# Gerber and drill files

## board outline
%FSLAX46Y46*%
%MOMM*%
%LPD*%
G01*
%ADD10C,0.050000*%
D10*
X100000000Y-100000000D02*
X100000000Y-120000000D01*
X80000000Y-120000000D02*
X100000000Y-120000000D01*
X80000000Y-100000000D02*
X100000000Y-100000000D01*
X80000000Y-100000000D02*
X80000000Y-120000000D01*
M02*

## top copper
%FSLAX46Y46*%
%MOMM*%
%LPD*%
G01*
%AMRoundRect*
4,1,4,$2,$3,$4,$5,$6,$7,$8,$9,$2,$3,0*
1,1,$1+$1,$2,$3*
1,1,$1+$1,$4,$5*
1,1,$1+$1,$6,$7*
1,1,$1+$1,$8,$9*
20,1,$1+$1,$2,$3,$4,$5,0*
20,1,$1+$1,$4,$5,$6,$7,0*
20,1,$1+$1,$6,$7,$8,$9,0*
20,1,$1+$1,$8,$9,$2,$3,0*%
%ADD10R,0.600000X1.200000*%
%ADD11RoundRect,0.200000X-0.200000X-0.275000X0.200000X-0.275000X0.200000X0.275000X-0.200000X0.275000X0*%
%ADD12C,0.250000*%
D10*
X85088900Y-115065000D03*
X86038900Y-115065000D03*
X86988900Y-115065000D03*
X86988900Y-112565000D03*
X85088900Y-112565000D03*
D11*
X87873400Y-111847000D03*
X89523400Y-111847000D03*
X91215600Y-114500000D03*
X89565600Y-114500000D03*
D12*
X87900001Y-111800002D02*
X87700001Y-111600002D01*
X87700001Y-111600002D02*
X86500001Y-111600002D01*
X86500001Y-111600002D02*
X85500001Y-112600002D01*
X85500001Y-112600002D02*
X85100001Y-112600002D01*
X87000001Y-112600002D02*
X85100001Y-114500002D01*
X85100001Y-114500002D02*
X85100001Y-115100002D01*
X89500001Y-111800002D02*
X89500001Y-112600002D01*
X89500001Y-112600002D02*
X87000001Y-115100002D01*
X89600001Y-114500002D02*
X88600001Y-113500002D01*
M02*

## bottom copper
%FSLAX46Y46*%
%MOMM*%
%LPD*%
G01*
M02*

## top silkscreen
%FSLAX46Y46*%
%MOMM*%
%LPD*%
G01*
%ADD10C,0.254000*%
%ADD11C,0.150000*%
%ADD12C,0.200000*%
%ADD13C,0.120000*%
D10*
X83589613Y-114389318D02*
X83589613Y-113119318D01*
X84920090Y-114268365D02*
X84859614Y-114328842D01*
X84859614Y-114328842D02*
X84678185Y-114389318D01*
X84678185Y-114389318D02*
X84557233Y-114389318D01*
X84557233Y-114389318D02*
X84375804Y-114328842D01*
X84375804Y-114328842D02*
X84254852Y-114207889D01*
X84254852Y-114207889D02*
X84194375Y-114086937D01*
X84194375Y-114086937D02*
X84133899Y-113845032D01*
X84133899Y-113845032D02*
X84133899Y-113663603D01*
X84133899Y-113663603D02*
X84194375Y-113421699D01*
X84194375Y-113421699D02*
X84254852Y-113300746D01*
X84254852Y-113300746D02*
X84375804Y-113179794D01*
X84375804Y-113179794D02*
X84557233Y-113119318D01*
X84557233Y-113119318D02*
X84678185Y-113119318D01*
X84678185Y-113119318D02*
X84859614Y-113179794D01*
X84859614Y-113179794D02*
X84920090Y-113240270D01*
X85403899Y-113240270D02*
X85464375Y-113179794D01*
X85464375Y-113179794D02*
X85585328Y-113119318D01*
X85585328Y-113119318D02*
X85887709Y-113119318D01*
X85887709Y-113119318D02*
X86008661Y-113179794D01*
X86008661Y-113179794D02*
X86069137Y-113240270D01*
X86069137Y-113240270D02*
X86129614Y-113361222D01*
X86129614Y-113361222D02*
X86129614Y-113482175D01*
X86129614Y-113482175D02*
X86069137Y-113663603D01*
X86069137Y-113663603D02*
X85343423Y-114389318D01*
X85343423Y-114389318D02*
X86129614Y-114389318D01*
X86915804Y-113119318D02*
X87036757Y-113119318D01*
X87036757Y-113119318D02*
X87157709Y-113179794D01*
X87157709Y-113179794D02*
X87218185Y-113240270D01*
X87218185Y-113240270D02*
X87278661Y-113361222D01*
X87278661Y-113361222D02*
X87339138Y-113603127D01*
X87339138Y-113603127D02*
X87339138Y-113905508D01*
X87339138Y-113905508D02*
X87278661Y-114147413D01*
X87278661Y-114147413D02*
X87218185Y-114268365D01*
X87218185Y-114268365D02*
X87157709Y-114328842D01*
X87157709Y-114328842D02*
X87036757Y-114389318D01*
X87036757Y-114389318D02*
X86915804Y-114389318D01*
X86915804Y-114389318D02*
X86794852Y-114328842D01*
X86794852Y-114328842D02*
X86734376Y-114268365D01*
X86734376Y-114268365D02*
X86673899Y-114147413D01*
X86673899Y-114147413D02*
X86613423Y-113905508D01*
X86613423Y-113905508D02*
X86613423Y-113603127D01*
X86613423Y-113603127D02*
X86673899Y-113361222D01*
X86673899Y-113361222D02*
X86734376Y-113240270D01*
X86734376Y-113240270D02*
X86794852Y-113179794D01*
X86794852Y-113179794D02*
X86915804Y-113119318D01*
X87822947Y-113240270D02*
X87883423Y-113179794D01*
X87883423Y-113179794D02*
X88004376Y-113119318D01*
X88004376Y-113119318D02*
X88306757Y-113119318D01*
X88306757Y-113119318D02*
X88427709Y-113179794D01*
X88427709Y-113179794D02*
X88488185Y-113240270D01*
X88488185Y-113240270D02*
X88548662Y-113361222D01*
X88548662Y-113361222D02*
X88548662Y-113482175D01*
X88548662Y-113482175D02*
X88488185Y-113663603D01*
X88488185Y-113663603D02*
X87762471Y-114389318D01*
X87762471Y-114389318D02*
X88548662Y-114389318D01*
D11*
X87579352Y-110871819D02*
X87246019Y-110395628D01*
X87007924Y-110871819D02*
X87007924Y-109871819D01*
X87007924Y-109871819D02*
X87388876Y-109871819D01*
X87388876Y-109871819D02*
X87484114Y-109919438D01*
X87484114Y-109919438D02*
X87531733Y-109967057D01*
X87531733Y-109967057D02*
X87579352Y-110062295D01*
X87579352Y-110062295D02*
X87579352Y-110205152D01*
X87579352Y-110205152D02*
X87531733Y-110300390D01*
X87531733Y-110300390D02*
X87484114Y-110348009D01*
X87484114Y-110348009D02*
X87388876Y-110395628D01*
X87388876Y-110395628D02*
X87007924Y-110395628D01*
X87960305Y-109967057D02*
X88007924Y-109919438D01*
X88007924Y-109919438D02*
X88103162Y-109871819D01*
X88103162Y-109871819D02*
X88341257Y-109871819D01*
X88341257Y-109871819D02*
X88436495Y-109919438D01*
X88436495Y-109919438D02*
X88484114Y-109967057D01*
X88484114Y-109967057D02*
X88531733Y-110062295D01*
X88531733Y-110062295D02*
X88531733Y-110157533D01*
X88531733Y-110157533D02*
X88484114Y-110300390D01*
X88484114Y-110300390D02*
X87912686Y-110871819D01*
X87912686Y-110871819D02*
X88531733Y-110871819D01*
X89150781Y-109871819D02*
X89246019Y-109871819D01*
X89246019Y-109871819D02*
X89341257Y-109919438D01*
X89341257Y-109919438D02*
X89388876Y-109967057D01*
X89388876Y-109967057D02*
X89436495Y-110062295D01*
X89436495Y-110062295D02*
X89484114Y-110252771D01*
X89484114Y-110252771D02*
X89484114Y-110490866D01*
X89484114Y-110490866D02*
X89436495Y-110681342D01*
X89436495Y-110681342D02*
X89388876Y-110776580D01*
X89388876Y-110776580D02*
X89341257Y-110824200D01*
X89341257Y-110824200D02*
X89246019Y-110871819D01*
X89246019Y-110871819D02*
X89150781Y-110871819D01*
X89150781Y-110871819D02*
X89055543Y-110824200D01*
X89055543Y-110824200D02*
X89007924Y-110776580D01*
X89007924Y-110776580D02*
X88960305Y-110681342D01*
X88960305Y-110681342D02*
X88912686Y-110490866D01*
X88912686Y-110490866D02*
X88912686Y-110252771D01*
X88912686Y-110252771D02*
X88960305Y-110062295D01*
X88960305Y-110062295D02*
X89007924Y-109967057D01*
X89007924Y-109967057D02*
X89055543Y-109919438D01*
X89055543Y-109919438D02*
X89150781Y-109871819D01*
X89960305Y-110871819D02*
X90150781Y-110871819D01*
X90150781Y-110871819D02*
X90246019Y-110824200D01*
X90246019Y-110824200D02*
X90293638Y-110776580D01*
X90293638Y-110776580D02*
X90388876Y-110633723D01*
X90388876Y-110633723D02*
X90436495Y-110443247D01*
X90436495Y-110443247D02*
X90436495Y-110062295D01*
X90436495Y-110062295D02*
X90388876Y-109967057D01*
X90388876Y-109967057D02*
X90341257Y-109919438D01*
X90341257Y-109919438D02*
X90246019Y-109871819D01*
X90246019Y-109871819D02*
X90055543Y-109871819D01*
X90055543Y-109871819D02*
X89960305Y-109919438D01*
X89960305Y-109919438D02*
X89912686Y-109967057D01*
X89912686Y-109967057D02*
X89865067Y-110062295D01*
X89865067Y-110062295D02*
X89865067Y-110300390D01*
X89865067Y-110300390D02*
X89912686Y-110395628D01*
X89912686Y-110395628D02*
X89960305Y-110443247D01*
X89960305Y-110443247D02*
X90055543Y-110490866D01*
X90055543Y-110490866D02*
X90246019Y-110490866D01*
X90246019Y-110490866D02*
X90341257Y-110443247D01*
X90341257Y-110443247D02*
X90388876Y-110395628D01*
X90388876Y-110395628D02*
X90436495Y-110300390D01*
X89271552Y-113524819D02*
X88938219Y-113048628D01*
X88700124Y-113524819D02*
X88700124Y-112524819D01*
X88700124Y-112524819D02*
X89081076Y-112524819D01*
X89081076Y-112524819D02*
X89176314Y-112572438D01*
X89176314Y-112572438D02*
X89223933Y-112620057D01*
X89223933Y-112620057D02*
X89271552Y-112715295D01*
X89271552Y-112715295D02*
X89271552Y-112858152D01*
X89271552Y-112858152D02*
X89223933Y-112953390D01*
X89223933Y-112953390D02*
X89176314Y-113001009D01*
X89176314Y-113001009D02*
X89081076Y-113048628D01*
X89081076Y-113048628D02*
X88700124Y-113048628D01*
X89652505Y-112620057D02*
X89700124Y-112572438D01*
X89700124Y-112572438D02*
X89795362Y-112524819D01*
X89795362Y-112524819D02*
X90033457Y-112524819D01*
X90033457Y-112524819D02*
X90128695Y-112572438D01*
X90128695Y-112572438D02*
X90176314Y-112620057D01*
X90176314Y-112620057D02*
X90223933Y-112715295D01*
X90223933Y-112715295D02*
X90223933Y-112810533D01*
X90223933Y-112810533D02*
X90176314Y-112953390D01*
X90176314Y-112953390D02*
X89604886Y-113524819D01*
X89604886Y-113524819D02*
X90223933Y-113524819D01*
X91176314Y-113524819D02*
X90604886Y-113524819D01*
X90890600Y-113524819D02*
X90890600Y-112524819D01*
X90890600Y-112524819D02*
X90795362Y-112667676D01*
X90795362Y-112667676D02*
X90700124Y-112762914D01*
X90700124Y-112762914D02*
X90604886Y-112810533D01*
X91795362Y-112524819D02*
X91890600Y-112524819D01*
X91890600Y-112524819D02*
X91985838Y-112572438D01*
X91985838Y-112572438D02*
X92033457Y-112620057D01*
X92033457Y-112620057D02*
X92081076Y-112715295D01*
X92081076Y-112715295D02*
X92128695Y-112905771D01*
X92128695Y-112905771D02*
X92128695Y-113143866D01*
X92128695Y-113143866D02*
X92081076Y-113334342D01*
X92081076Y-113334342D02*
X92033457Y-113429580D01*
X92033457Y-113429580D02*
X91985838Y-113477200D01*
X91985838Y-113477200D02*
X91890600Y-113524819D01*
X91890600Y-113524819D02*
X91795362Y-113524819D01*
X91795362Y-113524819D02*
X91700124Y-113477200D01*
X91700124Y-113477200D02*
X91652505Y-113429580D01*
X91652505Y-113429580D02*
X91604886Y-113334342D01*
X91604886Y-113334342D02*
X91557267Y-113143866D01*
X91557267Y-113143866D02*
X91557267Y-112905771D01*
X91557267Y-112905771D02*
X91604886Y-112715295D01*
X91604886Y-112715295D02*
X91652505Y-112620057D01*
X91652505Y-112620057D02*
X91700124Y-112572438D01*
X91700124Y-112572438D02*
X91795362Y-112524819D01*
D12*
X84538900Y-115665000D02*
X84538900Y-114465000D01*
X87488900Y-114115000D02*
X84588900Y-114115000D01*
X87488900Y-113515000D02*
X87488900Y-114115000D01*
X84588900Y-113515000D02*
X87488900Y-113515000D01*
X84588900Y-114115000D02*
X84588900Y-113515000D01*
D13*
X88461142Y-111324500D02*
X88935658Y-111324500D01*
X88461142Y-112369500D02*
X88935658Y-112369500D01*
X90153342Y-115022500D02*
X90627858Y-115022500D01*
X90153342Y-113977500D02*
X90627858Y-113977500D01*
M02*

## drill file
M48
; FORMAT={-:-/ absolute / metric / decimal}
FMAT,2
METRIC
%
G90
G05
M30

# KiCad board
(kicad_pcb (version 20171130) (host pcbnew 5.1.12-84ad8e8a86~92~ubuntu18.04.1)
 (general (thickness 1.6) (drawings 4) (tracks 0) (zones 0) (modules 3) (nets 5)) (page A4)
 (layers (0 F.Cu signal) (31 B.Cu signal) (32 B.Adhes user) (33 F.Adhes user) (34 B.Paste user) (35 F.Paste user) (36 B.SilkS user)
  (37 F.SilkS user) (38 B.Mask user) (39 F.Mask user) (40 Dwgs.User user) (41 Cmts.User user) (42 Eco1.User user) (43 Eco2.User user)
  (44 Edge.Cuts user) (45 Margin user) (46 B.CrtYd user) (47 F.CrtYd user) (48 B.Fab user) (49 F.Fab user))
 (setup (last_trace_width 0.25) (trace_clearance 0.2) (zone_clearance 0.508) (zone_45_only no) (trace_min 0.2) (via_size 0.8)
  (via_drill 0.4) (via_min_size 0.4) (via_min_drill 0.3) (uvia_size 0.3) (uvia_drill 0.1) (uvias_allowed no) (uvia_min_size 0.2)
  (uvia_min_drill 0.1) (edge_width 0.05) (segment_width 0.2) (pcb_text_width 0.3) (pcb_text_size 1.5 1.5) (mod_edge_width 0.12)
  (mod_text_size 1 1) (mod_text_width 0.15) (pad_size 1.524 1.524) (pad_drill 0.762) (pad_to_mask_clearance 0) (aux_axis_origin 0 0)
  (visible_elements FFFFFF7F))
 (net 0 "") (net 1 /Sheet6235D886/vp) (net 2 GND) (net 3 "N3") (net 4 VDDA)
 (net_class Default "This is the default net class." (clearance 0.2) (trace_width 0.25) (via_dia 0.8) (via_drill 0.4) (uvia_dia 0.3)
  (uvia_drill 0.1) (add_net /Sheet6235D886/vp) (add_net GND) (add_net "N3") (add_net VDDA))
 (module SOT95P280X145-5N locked (layer F.Cu) (at 86.038900 113.815000 90.000000)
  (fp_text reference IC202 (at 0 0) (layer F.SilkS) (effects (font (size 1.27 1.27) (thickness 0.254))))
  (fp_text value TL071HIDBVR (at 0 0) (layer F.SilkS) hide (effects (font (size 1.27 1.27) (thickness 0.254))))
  (fp_line (start -1.85 -1.5) (end -0.65 -1.5) (layer F.SilkS) (width 0.2))
  (fp_line (start -0.3 1.45) (end -0.3 -1.45) (layer F.SilkS) (width 0.2))
  (fp_line (start 0.3 1.45) (end -0.3 1.45) (layer F.SilkS) (width 0.2))
  (fp_line (start 0.3 -1.45) (end 0.3 1.45) (layer F.SilkS) (width 0.2))
  (fp_line (start -0.3 -1.45) (end 0.3 -1.45) (layer F.SilkS) (width 0.2))
  (pad 1 smd rect (at -1.25 -0.95 180.000000) (size 0.6 1.2) (layers F.Cu F.Mask F.Paste) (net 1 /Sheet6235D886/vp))
  (pad 2 smd rect (at -1.25 0 180.000000) (size 0.6 1.2) (layers F.Cu F.Mask F.Paste) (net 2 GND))
  (pad 3 smd rect (at -1.25 0.95 180.000000) (size 0.6 1.2) (layers F.Cu F.Mask F.Paste) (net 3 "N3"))
  (pad 4 smd rect (at 1.25 0.95 180.000000) (size 0.6 1.2) (layers F.Cu F.Mask F.Paste) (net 1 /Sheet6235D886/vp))
  (pad 5 smd rect (at 1.25 -0.95 180.000000) (size 0.6 1.2) (layers F.Cu F.Mask F.Paste) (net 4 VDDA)))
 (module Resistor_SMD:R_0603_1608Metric (layer F.Cu) (at 88.698400 111.847000)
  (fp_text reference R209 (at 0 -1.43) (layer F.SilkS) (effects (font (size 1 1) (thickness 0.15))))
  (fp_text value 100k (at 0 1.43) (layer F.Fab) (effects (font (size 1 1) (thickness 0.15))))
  (fp_line (start -0.237258 -0.5225) (end 0.237258 -0.5225) (layer F.SilkS) (width 0.12))
  (fp_line (start -0.237258 0.5225) (end 0.237258 0.5225) (layer F.SilkS) (width 0.12))
  (pad 1 smd roundrect (at -0.825 0) (size 0.8 0.95) (layers F.Cu F.Mask F.Paste) (roundrect_rratio 0.25) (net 4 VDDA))
  (pad 2 smd roundrect (at 0.825 0) (size 0.8 0.95) (layers F.Cu F.Mask F.Paste) (roundrect_rratio 0.25) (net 3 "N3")))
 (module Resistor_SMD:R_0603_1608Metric (layer F.Cu) (at 90.390600 114.500000)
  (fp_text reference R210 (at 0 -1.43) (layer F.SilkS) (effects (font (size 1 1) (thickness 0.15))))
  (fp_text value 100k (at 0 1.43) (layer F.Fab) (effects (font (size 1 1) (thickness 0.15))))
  (fp_line (start -0.237258 0.5225) (end 0.237258 0.5225) (layer F.SilkS) (width 0.12))
  (fp_line (start -0.237258 -0.5225) (end 0.237258 -0.5225) (layer F.SilkS) (width 0.12))
  (pad 2 smd roundrect (at 0.825 0) (size 0.8 0.95) (layers F.Cu F.Mask F.Paste) (roundrect_rratio 0.25) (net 2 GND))
  (pad 1 smd roundrect (at -0.825 0) (size 0.8 0.95) (layers F.Cu F.Mask F.Paste) (roundrect_rratio 0.25) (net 3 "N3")))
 (gr_line (start 100 100) (end 100 120) (layer Edge.Cuts) (width 0.05))
 (gr_line (start 80 120) (end 100 120) (layer Edge.Cuts) (width 0.05))
 (gr_line (start 80 100) (end 100 100) (layer Edge.Cuts) (width 0.05))
 (gr_line (start 80 100) (end 80 120) (layer Edge.Cuts) (width 0.05))
 (segment (start 87.900001 111.800002) (end 87.700001 111.600002) (width 0.250000) (layer F.Cu) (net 4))
 (segment (start 87.700001 111.600002) (end 86.500001 111.600002) (width 0.250000) (layer F.Cu) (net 4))
 (segment (start 86.500001 111.600002) (end 85.500001 112.600002) (width 0.250000) (layer F.Cu) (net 4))
 (segment (start 85.500001 112.600002) (end 85.100001 112.600002) (width 0.250000) (layer F.Cu) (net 4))
 (segment (start 87.000001 112.600002) (end 85.100001 114.500002) (width 0.250000) (layer F.Cu) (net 1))
 (segment (start 85.100001 114.500002) (end 85.100001 115.100002) (width 0.250000) (layer F.Cu) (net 1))
 (segment (start 89.500001 111.800002) (end 89.500001 112.600002) (width 0.250000) (layer F.Cu) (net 3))
 (segment (start 89.500001 112.600002) (end 87.000001 115.100002) (width 0.250000) (layer F.Cu) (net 3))
 (segment (start 89.600001 114.500002) (end 88.600001 113.500002) (width 0.250000) (layer F.Cu) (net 3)))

